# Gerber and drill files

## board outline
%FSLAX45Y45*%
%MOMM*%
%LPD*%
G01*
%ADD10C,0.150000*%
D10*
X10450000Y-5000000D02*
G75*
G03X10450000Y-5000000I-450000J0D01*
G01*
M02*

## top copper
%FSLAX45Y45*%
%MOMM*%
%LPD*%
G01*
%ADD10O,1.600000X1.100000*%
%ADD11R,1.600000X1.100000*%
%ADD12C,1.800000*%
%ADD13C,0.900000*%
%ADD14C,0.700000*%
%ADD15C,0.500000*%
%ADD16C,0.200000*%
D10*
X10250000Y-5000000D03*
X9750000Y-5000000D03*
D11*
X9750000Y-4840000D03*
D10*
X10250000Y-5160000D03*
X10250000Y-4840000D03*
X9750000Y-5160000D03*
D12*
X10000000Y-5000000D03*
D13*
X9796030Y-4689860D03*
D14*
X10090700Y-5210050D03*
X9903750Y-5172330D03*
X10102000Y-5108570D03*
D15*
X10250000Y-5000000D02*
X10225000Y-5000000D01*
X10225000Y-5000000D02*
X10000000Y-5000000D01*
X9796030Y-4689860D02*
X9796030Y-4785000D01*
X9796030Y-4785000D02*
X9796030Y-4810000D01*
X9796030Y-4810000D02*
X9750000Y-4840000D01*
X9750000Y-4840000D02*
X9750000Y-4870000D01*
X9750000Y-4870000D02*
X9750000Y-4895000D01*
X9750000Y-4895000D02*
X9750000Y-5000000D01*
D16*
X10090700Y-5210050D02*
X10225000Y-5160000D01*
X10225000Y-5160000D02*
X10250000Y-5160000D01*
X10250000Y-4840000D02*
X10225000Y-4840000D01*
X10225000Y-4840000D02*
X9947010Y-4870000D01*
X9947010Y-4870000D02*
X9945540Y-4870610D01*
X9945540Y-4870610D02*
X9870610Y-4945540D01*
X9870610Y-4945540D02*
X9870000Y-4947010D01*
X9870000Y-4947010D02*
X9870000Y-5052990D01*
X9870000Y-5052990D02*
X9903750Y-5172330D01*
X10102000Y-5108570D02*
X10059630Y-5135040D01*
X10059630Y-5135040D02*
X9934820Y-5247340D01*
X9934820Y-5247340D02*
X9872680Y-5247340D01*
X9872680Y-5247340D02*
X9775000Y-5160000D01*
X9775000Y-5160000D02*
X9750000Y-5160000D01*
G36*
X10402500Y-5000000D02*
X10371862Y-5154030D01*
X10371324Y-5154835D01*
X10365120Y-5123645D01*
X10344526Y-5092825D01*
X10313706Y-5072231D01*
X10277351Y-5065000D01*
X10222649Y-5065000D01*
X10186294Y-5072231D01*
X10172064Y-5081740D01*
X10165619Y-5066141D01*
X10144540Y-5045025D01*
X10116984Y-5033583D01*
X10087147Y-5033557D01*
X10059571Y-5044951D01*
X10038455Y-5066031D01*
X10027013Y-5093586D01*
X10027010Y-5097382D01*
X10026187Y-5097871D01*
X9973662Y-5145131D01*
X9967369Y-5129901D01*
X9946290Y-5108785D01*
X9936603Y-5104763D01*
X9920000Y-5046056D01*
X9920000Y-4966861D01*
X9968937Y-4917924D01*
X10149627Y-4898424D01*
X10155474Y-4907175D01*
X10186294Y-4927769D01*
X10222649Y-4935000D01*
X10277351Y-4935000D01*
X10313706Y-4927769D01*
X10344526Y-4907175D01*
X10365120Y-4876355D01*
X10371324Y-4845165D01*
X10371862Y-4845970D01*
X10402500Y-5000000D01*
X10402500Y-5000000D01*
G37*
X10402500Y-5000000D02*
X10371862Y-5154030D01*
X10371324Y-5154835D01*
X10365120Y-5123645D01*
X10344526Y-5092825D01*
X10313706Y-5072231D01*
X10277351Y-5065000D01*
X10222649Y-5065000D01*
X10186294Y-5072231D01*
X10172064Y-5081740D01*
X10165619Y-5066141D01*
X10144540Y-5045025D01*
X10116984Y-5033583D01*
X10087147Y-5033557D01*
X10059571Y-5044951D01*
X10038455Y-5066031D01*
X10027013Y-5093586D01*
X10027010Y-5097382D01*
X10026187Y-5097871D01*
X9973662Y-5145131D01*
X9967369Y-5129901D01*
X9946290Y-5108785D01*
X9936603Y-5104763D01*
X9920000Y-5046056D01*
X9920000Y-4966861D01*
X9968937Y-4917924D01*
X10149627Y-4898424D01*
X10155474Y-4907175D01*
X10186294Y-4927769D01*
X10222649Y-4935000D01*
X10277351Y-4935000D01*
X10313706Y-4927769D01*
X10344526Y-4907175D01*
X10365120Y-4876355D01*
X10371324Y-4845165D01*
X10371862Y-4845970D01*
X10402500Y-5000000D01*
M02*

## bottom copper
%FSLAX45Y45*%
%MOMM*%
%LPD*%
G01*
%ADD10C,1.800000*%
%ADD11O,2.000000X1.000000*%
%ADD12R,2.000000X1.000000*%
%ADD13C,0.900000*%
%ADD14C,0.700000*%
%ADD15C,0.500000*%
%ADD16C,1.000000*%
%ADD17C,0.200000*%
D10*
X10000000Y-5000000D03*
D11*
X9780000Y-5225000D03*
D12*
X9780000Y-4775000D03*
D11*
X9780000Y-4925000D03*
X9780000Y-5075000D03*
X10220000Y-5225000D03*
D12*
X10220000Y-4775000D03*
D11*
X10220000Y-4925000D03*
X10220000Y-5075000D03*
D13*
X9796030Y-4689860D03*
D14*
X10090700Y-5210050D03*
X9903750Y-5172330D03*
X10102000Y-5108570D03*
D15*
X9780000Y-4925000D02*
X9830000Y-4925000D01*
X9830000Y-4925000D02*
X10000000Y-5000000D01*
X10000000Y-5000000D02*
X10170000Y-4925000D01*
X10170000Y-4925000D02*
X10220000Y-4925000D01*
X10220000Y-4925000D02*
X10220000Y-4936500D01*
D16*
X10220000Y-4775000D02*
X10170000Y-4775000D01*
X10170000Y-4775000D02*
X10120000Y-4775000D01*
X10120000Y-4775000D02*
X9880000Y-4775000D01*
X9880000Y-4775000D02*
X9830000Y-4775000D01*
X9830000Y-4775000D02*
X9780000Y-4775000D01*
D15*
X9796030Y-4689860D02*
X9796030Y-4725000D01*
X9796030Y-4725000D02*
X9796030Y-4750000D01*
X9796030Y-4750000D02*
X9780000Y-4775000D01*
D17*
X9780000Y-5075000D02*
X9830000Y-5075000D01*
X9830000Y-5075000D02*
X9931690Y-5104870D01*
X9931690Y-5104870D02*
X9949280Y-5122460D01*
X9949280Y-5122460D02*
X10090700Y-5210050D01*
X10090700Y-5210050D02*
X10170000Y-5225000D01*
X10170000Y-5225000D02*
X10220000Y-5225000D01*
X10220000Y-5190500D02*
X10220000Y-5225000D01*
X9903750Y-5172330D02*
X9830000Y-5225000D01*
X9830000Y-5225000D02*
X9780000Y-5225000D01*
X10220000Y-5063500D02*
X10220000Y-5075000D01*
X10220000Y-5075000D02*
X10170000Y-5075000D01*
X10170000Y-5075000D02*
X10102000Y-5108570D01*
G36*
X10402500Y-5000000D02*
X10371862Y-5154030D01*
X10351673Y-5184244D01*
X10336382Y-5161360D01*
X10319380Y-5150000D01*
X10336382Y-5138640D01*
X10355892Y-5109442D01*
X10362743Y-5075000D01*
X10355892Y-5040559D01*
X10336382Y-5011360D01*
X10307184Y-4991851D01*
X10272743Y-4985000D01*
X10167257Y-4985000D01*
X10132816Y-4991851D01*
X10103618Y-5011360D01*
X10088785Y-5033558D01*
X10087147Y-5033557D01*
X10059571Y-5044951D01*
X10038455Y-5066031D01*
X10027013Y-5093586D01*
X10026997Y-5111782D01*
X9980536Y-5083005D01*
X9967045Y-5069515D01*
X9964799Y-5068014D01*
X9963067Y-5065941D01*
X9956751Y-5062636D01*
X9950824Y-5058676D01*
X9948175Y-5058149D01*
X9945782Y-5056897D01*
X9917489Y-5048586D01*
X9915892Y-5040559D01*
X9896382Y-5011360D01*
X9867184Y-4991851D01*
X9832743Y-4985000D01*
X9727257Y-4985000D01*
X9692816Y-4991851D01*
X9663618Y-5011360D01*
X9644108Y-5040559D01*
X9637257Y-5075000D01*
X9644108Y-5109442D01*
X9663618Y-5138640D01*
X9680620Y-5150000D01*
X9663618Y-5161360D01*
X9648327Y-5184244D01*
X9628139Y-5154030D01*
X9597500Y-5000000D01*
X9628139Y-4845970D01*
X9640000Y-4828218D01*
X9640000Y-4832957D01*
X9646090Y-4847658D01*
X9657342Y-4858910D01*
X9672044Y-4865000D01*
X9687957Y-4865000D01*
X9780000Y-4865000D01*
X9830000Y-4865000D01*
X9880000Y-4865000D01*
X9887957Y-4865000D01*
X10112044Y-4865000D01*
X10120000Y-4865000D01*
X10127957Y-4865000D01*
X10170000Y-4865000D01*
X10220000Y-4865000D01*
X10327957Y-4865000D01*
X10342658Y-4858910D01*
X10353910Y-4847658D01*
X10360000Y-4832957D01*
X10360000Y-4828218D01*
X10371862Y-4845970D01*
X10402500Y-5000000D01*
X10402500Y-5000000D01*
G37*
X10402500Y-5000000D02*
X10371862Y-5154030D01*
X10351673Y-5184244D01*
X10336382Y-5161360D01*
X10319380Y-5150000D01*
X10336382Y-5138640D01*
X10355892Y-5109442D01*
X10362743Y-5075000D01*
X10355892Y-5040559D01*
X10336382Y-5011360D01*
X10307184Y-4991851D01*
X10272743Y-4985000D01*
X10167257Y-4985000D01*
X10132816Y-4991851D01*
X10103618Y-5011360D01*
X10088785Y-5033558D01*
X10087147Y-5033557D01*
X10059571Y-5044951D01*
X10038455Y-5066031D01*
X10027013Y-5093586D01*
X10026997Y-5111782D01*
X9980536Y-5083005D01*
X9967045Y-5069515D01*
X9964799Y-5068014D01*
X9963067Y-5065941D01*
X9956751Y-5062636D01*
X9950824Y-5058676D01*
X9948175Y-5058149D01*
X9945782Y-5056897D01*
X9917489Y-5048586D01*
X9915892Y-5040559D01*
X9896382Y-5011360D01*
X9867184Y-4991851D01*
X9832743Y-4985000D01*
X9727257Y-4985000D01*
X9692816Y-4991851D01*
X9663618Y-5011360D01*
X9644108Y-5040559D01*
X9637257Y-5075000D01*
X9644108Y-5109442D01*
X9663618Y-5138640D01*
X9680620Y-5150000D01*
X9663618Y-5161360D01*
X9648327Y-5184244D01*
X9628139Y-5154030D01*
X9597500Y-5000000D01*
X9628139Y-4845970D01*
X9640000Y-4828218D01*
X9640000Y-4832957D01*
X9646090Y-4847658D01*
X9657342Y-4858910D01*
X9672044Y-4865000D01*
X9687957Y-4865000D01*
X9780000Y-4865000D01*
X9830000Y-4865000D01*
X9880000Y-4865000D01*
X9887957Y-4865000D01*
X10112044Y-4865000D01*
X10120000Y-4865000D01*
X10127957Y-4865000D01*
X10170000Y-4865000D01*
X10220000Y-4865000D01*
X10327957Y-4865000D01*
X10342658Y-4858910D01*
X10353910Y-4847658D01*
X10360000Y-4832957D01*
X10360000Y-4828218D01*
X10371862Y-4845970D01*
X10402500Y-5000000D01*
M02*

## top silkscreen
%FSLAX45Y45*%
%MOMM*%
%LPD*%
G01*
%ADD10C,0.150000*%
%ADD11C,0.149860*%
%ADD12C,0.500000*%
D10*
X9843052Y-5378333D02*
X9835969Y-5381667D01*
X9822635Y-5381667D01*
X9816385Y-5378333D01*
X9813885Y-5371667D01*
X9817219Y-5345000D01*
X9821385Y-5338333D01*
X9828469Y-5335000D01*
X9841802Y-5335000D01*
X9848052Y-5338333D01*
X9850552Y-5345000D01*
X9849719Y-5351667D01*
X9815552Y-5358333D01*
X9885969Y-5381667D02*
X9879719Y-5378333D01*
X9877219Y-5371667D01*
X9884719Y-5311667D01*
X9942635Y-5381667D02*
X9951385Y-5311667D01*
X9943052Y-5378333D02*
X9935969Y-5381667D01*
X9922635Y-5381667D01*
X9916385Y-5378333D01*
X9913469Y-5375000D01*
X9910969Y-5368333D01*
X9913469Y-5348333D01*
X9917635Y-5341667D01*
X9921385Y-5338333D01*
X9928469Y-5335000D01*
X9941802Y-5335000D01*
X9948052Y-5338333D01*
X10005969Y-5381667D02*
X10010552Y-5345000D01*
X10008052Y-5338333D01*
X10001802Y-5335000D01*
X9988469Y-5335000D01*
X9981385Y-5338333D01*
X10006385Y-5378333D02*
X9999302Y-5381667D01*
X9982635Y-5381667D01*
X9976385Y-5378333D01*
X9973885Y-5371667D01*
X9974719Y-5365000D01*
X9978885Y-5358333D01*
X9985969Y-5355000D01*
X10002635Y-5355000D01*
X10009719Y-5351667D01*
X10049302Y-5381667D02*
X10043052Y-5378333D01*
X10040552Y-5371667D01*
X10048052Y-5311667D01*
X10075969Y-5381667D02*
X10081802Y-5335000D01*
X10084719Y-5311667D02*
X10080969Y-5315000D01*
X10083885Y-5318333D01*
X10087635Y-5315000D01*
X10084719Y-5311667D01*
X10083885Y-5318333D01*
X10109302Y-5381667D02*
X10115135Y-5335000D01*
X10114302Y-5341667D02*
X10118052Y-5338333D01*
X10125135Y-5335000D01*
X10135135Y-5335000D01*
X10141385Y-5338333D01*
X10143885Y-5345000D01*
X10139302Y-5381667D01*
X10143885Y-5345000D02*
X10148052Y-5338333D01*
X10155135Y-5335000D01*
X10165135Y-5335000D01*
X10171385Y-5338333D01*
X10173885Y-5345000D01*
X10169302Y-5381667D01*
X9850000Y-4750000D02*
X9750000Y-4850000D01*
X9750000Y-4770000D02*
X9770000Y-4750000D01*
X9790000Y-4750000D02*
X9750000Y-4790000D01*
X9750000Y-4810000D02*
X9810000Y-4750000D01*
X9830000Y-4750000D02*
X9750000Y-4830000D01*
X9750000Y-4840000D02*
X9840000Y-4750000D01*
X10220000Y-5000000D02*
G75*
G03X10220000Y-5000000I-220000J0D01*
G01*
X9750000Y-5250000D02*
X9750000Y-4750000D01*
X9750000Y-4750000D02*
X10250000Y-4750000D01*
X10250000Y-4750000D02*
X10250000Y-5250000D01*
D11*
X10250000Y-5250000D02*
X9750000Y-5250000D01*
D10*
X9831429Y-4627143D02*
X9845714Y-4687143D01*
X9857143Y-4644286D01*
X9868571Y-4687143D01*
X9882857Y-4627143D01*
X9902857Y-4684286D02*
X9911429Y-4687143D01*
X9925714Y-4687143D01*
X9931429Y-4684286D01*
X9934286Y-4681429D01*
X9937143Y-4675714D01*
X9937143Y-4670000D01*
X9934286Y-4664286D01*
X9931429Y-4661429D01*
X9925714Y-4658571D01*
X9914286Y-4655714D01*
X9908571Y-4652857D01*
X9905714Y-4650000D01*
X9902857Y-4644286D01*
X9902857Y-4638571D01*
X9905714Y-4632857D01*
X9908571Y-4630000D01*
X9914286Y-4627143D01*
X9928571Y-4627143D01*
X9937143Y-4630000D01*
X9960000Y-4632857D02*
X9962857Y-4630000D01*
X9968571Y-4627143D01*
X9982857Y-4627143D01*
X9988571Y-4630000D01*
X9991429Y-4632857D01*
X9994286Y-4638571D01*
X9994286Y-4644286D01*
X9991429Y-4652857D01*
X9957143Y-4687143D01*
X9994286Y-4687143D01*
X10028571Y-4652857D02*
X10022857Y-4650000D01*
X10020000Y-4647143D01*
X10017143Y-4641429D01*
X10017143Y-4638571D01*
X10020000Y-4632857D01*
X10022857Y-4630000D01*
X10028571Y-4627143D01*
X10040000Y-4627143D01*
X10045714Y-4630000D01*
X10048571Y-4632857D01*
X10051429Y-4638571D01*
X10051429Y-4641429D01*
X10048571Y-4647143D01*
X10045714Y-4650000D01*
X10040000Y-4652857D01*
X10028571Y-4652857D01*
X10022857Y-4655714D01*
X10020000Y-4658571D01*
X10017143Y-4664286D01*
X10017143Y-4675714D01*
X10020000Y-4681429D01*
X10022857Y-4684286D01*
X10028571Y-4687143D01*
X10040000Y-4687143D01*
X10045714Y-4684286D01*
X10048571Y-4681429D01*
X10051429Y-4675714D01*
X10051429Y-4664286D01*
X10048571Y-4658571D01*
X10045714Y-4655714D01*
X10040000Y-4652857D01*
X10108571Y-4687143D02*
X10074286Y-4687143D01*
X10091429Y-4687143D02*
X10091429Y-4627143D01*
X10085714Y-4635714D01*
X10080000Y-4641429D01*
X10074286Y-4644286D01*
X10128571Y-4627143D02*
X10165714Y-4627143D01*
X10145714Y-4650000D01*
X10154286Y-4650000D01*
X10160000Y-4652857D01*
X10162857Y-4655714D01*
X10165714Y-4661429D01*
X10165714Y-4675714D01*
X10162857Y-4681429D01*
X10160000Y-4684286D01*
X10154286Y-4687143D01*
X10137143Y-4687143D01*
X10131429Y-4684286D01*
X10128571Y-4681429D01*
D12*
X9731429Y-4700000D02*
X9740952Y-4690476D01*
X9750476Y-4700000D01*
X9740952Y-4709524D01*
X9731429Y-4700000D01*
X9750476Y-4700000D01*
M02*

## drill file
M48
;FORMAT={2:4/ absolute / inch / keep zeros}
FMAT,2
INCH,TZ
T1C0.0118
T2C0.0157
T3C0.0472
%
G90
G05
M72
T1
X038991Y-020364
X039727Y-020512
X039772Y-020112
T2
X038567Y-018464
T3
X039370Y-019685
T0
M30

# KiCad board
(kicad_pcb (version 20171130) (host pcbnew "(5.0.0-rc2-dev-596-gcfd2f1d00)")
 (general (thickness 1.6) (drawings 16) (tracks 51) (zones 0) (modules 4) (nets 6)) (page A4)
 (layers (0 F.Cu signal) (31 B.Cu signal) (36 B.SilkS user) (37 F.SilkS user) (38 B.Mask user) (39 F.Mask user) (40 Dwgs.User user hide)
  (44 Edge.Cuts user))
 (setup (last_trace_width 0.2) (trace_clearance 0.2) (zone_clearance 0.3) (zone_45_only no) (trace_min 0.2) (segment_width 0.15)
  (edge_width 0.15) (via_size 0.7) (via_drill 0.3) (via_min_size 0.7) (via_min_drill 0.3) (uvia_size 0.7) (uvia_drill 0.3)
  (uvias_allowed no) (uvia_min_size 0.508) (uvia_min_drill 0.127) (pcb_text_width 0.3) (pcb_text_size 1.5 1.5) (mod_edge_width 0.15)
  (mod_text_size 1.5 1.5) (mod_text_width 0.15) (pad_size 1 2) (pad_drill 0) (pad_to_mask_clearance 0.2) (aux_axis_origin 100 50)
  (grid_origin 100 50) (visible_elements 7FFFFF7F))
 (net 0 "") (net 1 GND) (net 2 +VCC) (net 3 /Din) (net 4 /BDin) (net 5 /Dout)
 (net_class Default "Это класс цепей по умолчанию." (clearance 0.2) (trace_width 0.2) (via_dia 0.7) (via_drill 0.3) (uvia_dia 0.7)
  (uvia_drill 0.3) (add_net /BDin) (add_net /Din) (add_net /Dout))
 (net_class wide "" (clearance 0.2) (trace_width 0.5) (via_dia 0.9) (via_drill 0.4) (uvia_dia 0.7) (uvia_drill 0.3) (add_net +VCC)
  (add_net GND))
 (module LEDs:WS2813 (layer F.Cu) (at 100 50 180)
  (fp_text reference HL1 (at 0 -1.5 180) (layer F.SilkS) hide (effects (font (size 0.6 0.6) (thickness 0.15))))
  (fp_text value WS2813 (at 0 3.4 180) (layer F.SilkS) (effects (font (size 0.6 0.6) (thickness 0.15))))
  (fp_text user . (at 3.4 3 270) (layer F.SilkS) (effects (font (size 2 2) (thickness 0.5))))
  (fp_line (start 1.5 2.5) (end 2.5 1.5) (layer F.SilkS) (width 0.15))
  (fp_line (start 2.5 2.3) (end 2.3 2.5) (layer F.SilkS) (width 0.15))
  (fp_line (start 2.1 2.5) (end 2.5 2.1) (layer F.SilkS) (width 0.15))
  (fp_line (start 2.5 1.9) (end 1.9 2.5) (layer F.SilkS) (width 0.15))
  (fp_line (start 1.7 2.5) (end 2.5 1.7) (layer F.SilkS) (width 0.15))
  (fp_line (start 2.5 1.6) (end 1.6 2.5) (layer F.SilkS) (width 0.15))
  (fp_circle (center 0 0) (end 0 2.2) (layer F.SilkS) (width 0.15))
  (fp_line (start 2.5 -2.5) (end 2.5 2.5) (layer F.SilkS) (width 0.15))
  (fp_line (start 2.5 2.5) (end -2.5 2.5) (layer F.SilkS) (width 0.15))
  (fp_line (start -2.5 2.5) (end -2.5 -2.5) (layer F.SilkS) (width 0.15))
  (fp_line (start -2.5 -2.5) (end 2.5 -2.5) (layer F.SilkS) (width 0.14986))
  (pad 5 smd oval (at -2.5 0 180) (size 1.6 1.1) (layers F.Cu F.Mask) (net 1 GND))
  (pad 2 smd oval (at 2.5 0 180) (size 1.6 1.1) (layers F.Cu F.Mask) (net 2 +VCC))
  (pad 1 smd rect (at 2.5 1.6 180) (size 1.6 1.1) (layers F.Cu F.Mask) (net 2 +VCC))
  (pad 4 smd oval (at -2.5 -1.6 180) (size 1.6 1.1) (layers F.Cu F.Mask) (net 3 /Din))
  (pad 6 smd oval (at -2.5 1.6 180) (size 1.6 1.1) (layers F.Cu F.Mask) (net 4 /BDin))
  (pad 3 smd oval (at 2.5 -1.6 180) (size 1.6 1.1) (layers F.Cu F.Mask) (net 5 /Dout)))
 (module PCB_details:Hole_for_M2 (layer F.Cu) (at 100 50 270)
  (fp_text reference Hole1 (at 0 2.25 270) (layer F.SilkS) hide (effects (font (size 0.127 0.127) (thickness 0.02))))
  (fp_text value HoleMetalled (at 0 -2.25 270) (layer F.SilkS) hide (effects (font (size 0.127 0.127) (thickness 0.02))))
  (pad H thru_hole circle (at 0 0 270) (size 1.8 1.8) (drill 1.2) (layers *.Cu *.Mask) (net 1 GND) (zone_connect 2)))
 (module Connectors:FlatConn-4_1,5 (layer B.Cu) (at 97.8 50 270)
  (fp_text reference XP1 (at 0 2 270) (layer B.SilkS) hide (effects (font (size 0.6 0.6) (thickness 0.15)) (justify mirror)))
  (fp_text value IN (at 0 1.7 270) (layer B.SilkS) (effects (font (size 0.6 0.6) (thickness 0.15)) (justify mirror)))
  (pad 4 smd oval (at 2.25 0 270) (size 1 2) (layers B.Cu B.Mask) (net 4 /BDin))
  (pad 1 smd rect (at -2.25 0 270) (size 1 2) (layers B.Cu B.Mask) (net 2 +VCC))
  (pad 2 smd oval (at -0.75 0 270) (size 1 2) (layers B.Cu B.Mask) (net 1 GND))
  (pad 3 smd oval (at 0.75 0 270) (size 1 2) (layers B.Cu B.Mask) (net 3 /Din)))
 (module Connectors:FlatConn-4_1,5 (layer B.Cu) (at 102.2 50 270)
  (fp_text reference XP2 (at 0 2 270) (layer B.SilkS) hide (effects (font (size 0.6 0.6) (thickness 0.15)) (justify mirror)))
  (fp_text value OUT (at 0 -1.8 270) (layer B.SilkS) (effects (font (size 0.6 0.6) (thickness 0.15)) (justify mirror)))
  (pad 4 smd oval (at 2.25 0 270) (size 1 2) (layers B.Cu B.Mask) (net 3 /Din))
  (pad 1 smd rect (at -2.25 0 270) (size 1 2) (layers B.Cu B.Mask) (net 2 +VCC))
  (pad 2 smd oval (at -0.75 0 270) (size 1 2) (layers B.Cu B.Mask) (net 1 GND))
  (pad 3 smd oval (at 0.75 0 270) (size 1 2) (layers B.Cu B.Mask) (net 5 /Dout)))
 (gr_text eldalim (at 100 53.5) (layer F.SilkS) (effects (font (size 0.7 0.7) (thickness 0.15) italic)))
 (gr_circle (center 100 50) (end 95.5 50) (layer Edge.Cuts) (width 0.15))
 (segment (start 102.5 50) (end 102.25 50) (width 0.5) (layer F.Cu) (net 1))
 (segment (start 102.25 50) (end 100 50) (width 0.5) (layer F.Cu) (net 1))
 (segment (start 97.8 49.25) (end 98.3 49.25) (width 0.5) (layer B.Cu) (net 1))
 (segment (start 98.3 49.25) (end 100 50) (width 0.5) (layer B.Cu) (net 1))
 (segment (start 100 50) (end 101.7 49.25) (width 0.5) (layer B.Cu) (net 1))
 (segment (start 101.7 49.25) (end 102.2 49.25) (width 0.5) (layer B.Cu) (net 1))
 (segment (start 102.2 49.25) (end 102.2 49.365) (width 0.5) (layer B.Cu) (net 1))
 (segment (start 97.9603 46.8986) (end 97.9603 47.85) (width 0.5) (layer F.Cu) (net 2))
 (segment (start 97.9603 47.85) (end 97.9603 48.1) (width 0.5) (layer F.Cu) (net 2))
 (segment (start 97.9603 48.1) (end 97.5 48.4) (width 0.5) (layer F.Cu) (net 2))
 (segment (start 97.5 48.4) (end 97.5 48.7) (width 0.5) (layer F.Cu) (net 2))
 (segment (start 97.5 48.7) (end 97.5 48.95) (width 0.5) (layer F.Cu) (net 2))
 (segment (start 97.5 48.95) (end 97.5 50) (width 0.5) (layer F.Cu) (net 2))
 (segment (start 102.2 47.75) (end 101.7 47.75) (width 1) (layer B.Cu) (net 2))
 (segment (start 101.7 47.75) (end 101.2 47.75) (width 1) (layer B.Cu) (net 2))
 (segment (start 101.2 47.75) (end 98.8 47.75) (width 1) (layer B.Cu) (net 2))
 (segment (start 98.8 47.75) (end 98.3 47.75) (width 1) (layer B.Cu) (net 2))
 (segment (start 98.3 47.75) (end 97.8 47.75) (width 1) (layer B.Cu) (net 2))
 (segment (start 97.9603 46.8986) (end 97.9603 47.25) (width 0.5) (layer B.Cu) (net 2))
 (segment (start 97.9603 47.25) (end 97.9603 47.5) (width 0.5) (layer B.Cu) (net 2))
 (segment (start 97.9603 47.5) (end 97.8 47.75) (width 0.5) (layer B.Cu) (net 2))
 (via (at 97.9603 46.8986) (size 0.9) (layers F.Cu B.Cu) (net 2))
 (segment (start 100.907 52.1005) (end 102.25 51.6) (width 0.2) (layer F.Cu) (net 3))
 (segment (start 102.25 51.6) (end 102.5 51.6) (width 0.2) (layer F.Cu) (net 3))
 (segment (start 97.8 50.75) (end 98.3 50.75) (width 0.2) (layer B.Cu) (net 3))
 (segment (start 98.3 50.75) (end 99.3169 51.0487) (width 0.2) (layer B.Cu) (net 3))
 (segment (start 99.3169 51.0487) (end 99.4928 51.2246) (width 0.2) (layer B.Cu) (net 3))
 (segment (start 99.4928 51.2246) (end 100.907 52.1005) (width 0.2) (layer B.Cu) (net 3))
 (segment (start 100.907 52.1005) (end 101.7 52.25) (width 0.2) (layer B.Cu) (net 3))
 (segment (start 101.7 52.25) (end 102.2 52.25) (width 0.2) (layer B.Cu) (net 3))
 (segment (start 102.2 51.905) (end 102.2 52.25) (width 0.2) (layer B.Cu) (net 3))
 (via (at 100.907 52.1005) (size 0.7) (layers F.Cu B.Cu) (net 3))
 (segment (start 102.5 48.4) (end 102.25 48.4) (width 0.2) (layer F.Cu) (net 4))
 (segment (start 102.25 48.4) (end 99.4701 48.7) (width 0.2) (layer F.Cu) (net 4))
 (segment (start 99.4701 48.7) (end 99.4554 48.7061) (width 0.2) (layer F.Cu) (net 4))
 (segment (start 99.4554 48.7061) (end 98.7061 49.4554) (width 0.2) (layer F.Cu) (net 4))
 (segment (start 98.7061 49.4554) (end 98.7 49.4701) (width 0.2) (layer F.Cu) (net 4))
 (segment (start 98.7 49.4701) (end 98.7 50.5299) (width 0.2) (layer F.Cu) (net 4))
 (segment (start 98.7 50.5299) (end 99.0375 51.7233) (width 0.2) (layer F.Cu) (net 4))
 (segment (start 99.0375 51.7233) (end 98.3 52.25) (width 0.2) (layer B.Cu) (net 4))
 (segment (start 98.3 52.25) (end 97.8 52.25) (width 0.2) (layer B.Cu) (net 4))
 (via (at 99.0375 51.7233) (size 0.7) (layers F.Cu B.Cu) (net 4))
 (segment (start 101.02 51.0857) (end 100.5963 51.3504) (width 0.2) (layer F.Cu) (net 5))
 (segment (start 100.5963 51.3504) (end 99.3482 52.4734) (width 0.2) (layer F.Cu) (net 5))
 (segment (start 99.3482 52.4734) (end 98.7268 52.4734) (width 0.2) (layer F.Cu) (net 5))
 (segment (start 98.7268 52.4734) (end 97.75 51.6) (width 0.2) (layer F.Cu) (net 5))
 (segment (start 97.75 51.6) (end 97.5 51.6) (width 0.2) (layer F.Cu) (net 5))
 (segment (start 102.2 50.635) (end 102.2 50.75) (width 0.2) (layer B.Cu) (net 5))
 (segment (start 102.2 50.75) (end 101.7 50.75) (width 0.2) (layer B.Cu) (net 5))
 (segment (start 101.7 50.75) (end 101.02 51.0857) (width 0.2) (layer B.Cu) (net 5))
 (via (at 101.02 51.0857) (size 0.7) (layers F.Cu B.Cu) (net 5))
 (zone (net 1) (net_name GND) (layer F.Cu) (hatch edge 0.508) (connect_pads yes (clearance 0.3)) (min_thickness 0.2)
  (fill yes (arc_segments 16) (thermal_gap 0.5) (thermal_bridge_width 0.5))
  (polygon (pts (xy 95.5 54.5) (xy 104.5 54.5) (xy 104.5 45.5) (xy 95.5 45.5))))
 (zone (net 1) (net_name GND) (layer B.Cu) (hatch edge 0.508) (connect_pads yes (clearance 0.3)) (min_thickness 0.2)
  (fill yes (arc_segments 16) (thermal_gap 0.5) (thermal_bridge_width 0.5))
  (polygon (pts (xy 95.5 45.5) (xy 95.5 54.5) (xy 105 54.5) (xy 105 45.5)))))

